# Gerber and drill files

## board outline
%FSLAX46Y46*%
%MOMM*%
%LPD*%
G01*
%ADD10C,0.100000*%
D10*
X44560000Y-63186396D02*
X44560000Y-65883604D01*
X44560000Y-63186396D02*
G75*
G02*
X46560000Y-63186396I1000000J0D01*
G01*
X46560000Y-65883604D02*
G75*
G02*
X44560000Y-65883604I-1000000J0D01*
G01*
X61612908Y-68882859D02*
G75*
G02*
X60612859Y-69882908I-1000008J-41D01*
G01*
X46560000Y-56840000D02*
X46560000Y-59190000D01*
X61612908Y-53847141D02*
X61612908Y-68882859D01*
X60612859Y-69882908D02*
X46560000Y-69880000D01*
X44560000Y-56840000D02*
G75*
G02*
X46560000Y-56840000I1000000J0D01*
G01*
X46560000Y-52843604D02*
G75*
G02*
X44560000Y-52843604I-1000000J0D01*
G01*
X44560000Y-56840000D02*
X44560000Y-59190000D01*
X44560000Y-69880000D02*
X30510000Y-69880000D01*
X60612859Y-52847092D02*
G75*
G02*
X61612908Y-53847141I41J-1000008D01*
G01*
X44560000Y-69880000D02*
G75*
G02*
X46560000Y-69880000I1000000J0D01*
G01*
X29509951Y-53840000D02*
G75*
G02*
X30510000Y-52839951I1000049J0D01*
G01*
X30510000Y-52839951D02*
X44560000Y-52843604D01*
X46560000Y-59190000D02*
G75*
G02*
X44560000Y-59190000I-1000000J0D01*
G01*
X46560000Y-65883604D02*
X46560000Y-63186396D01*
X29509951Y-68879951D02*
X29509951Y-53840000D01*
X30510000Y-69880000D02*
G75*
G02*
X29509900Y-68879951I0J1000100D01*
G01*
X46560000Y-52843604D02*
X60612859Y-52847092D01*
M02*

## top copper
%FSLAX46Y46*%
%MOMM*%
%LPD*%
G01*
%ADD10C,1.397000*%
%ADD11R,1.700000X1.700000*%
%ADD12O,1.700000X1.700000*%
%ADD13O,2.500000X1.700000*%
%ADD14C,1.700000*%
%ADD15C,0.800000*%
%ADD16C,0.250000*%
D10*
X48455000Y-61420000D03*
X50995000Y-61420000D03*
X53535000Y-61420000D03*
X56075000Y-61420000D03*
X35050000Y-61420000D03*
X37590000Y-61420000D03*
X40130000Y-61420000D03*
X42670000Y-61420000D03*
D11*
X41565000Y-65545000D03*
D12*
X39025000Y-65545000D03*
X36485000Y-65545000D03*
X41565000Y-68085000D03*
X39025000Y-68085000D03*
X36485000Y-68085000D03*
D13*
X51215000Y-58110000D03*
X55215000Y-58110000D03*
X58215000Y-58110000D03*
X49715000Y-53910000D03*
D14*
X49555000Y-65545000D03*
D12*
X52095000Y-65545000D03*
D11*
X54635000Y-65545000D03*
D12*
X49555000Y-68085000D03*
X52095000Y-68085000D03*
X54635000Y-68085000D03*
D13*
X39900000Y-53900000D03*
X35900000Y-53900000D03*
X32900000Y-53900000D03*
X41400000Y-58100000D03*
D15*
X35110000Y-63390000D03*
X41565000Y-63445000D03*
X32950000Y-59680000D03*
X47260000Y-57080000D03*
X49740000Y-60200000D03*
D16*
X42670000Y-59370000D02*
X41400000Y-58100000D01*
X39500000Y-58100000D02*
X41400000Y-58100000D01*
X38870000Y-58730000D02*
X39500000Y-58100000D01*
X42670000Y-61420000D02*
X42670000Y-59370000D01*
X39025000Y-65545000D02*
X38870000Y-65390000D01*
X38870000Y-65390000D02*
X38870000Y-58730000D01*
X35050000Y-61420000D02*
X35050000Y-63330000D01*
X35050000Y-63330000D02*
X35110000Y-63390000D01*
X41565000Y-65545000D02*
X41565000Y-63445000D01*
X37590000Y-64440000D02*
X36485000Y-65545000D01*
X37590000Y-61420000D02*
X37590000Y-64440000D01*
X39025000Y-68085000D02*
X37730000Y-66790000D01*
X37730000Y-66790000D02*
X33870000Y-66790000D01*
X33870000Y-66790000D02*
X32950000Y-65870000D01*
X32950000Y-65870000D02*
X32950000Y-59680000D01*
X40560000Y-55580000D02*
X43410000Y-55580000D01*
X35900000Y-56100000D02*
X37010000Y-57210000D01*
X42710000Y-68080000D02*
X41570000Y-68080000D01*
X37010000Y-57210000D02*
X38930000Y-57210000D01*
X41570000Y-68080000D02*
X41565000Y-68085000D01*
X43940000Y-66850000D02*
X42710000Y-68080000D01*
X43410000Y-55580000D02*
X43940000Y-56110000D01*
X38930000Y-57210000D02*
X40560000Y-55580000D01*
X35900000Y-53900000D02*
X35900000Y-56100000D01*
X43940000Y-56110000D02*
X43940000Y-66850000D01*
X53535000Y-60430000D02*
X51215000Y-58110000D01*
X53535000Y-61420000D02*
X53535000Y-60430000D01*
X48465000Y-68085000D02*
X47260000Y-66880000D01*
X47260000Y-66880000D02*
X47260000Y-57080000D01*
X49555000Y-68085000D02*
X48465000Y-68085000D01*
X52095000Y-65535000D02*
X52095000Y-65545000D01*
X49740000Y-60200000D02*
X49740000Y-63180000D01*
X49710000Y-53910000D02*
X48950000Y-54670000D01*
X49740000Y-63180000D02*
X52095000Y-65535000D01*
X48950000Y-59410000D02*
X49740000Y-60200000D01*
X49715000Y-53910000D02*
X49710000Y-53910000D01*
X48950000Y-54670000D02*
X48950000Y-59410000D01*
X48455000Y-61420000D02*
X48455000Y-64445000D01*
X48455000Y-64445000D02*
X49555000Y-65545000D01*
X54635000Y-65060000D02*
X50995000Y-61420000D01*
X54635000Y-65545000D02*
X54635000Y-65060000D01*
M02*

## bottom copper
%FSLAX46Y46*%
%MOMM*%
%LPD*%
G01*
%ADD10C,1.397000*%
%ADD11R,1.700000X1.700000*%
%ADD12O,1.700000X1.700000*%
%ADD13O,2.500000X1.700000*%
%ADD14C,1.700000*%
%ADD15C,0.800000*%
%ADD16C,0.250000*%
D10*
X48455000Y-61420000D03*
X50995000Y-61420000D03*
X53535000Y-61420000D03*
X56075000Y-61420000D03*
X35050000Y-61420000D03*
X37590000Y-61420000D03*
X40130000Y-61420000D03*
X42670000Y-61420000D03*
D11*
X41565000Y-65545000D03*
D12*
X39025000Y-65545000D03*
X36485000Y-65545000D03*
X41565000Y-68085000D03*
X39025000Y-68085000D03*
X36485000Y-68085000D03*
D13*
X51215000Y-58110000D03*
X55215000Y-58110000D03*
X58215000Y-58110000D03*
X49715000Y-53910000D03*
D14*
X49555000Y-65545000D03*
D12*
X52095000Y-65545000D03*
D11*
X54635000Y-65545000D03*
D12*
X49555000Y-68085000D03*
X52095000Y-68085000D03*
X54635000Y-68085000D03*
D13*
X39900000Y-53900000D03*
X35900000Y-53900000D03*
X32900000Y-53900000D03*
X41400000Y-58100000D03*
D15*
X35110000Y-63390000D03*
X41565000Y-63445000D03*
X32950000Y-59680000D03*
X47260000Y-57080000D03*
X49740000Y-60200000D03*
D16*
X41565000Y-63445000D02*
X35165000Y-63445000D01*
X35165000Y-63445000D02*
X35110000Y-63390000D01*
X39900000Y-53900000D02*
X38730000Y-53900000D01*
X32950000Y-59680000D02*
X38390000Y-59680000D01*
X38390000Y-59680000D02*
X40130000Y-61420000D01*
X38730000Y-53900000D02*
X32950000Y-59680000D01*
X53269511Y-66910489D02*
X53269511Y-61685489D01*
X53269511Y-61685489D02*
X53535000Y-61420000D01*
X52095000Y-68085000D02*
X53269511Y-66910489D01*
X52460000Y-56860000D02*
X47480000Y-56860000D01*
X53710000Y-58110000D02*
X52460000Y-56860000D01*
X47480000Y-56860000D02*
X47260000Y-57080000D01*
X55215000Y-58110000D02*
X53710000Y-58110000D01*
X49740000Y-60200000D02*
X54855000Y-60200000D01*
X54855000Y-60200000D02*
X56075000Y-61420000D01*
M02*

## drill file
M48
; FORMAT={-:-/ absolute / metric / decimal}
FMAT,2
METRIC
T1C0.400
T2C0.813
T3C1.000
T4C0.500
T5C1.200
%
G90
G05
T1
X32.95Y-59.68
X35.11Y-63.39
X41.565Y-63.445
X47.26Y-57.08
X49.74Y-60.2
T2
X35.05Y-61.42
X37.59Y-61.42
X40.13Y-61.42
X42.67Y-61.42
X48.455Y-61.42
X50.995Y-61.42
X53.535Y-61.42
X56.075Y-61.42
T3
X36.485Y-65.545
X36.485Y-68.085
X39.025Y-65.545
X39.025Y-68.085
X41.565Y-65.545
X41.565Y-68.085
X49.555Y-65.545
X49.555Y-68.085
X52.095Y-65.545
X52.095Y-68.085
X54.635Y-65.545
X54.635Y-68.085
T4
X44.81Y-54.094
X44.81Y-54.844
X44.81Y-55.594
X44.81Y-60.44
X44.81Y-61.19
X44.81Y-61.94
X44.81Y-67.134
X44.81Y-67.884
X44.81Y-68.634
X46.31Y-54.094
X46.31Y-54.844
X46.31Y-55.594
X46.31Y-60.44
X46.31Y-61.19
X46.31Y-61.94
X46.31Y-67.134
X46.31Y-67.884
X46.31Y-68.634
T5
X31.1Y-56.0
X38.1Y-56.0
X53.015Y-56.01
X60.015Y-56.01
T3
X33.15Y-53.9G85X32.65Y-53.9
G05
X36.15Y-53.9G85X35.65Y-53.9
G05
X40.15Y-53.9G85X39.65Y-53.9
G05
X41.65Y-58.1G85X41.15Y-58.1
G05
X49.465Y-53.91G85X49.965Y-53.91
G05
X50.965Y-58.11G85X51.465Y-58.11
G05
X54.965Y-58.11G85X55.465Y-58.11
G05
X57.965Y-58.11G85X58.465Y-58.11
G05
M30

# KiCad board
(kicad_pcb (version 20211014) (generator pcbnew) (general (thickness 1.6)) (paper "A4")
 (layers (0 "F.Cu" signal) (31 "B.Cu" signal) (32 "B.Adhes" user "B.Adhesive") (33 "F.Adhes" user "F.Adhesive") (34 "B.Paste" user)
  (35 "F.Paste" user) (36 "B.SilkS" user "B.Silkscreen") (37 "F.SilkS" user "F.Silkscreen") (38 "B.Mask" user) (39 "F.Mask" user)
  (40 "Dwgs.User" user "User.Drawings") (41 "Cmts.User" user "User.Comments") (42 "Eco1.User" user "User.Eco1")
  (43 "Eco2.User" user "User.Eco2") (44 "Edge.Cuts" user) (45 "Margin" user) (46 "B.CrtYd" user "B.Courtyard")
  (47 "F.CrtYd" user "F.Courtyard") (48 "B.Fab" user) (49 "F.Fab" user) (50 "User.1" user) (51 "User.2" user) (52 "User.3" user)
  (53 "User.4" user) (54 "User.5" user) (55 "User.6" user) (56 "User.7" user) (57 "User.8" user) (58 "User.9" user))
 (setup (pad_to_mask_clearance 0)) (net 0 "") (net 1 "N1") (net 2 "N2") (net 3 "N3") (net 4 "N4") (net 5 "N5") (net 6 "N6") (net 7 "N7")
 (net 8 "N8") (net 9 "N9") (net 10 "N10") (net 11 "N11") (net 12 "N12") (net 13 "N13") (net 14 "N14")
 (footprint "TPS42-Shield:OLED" (layer "F.Cu") (at 52.265 61.42)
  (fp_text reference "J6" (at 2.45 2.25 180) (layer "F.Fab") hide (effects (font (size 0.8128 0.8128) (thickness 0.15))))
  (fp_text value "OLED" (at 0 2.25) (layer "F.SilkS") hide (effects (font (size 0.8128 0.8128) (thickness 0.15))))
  (pad "1" thru_hole circle (at -3.81 0) (size 1.397 1.397) (drill 0.8128) (layers *.Cu *.Mask "F.SilkS") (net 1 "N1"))
  (pad "2" thru_hole circle (at -1.27 0) (size 1.397 1.397) (drill 0.8128) (layers *.Cu *.Mask "F.SilkS") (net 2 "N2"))
  (pad "3" thru_hole circle (at 1.27 0) (size 1.397 1.397) (drill 0.8128) (layers *.Cu *.Mask "F.SilkS") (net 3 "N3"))
  (pad "4" thru_hole circle (at 3.81 0) (size 1.397 1.397) (drill 0.8128) (layers *.Cu *.Mask "F.SilkS") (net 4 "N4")))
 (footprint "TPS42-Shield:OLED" (layer "F.Cu") (at 38.86 61.42)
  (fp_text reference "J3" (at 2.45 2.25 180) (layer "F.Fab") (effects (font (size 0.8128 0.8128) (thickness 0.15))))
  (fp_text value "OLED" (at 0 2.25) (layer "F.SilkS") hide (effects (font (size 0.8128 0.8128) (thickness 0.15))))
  (pad "1" thru_hole circle (at -3.81 0) (size 1.397 1.397) (drill 0.8128) (layers *.Cu *.Mask "F.SilkS") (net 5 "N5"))
  (pad "2" thru_hole circle (at -1.27 0) (size 1.397 1.397) (drill 0.8128) (layers *.Cu *.Mask "F.SilkS") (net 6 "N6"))
  (pad "3" thru_hole circle (at 1.27 0) (size 1.397 1.397) (drill 0.8128) (layers *.Cu *.Mask "F.SilkS") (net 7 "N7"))
  (pad "4" thru_hole circle (at 3.81 0) (size 1.397 1.397) (drill 0.8128) (layers *.Cu *.Mask "F.SilkS") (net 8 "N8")))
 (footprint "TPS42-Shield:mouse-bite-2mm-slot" (layer "F.Cu") (at 45.56 67.883604 90)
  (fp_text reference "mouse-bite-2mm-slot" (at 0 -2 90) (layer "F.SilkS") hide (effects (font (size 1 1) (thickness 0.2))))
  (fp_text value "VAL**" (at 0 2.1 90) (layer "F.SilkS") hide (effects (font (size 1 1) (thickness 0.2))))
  (pad "" np_thru_hole circle (at -0.75 0.75 90) (size 0.5 0.5) (drill 0.5) (layers *.Cu *.Mask))
  (pad "" np_thru_hole circle (at 0.75 -0.75 90) (size 0.5 0.5) (drill 0.5) (layers *.Cu *.Mask))
  (pad "" np_thru_hole circle (at -0.75 -0.75 90) (size 0.5 0.5) (drill 0.5) (layers *.Cu *.Mask))
  (pad "" np_thru_hole circle (at 0 -0.75 90) (size 0.5 0.5) (drill 0.5) (layers *.Cu *.Mask))
  (pad "" np_thru_hole circle (at 0.75 0.75 90) (size 0.5 0.5) (drill 0.5) (layers *.Cu *.Mask))
  (pad "" np_thru_hole circle (at 0 0.75 90) (size 0.5 0.5) (drill 0.5) (layers *.Cu *.Mask)))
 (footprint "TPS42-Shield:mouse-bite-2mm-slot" (layer "F.Cu") (at 45.56 61.19 90)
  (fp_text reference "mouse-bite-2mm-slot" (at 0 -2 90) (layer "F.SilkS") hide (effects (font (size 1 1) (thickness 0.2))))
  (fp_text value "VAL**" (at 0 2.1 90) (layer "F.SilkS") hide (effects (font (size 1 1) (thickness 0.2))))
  (pad "" np_thru_hole circle (at -0.75 0.75 90) (size 0.5 0.5) (drill 0.5) (layers *.Cu *.Mask))
  (pad "" np_thru_hole circle (at 0.75 -0.75 90) (size 0.5 0.5) (drill 0.5) (layers *.Cu *.Mask))
  (pad "" np_thru_hole circle (at -0.75 -0.75 90) (size 0.5 0.5) (drill 0.5) (layers *.Cu *.Mask))
  (pad "" np_thru_hole circle (at 0 -0.75 90) (size 0.5 0.5) (drill 0.5) (layers *.Cu *.Mask))
  (pad "" np_thru_hole circle (at 0.75 0.75 90) (size 0.5 0.5) (drill 0.5) (layers *.Cu *.Mask))
  (pad "" np_thru_hole circle (at 0 0.75 90) (size 0.5 0.5) (drill 0.5) (layers *.Cu *.Mask)))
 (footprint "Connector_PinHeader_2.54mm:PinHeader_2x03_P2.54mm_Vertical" (layer "F.Cu") (at 41.565 65.545 -90)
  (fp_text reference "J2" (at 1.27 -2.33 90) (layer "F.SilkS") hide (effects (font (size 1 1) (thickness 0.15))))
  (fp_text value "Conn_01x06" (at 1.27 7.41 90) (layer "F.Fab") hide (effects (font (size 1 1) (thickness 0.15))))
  (pad "1" thru_hole rect (at 0 0 270) (size 1.7 1.7) (drill 1) (layers *.Cu *.Mask) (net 5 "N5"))
  (pad "2" thru_hole oval (at 0 2.54 270) (size 1.7 1.7) (drill 1) (layers *.Cu *.Mask) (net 8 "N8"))
  (pad "3" thru_hole oval (at 0 5.08 270) (size 1.7 1.7) (drill 1) (layers *.Cu *.Mask) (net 6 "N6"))
  (pad "4" thru_hole oval (at 2.54 0 270) (size 1.7 1.7) (drill 1) (layers *.Cu *.Mask) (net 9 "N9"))
  (pad "5" thru_hole oval (at 2.54 2.54 270) (size 1.7 1.7) (drill 1) (layers *.Cu *.Mask) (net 7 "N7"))
  (pad "6" thru_hole oval (at 2.54 5.08 270) (size 1.7 1.7) (drill 1) (layers *.Cu *.Mask) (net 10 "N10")))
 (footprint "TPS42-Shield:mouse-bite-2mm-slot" (layer "F.Cu") (at 45.56 54.843604 90)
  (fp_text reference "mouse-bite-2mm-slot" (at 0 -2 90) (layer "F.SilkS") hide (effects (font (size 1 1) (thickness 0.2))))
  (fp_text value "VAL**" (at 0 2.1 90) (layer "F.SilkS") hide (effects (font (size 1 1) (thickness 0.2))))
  (pad "" np_thru_hole circle (at -0.75 0.75 90) (size 0.5 0.5) (drill 0.5) (layers *.Cu *.Mask))
  (pad "" np_thru_hole circle (at 0.75 -0.75 90) (size 0.5 0.5) (drill 0.5) (layers *.Cu *.Mask))
  (pad "" np_thru_hole circle (at -0.75 -0.75 90) (size 0.5 0.5) (drill 0.5) (layers *.Cu *.Mask))
  (pad "" np_thru_hole circle (at 0 -0.75 90) (size 0.5 0.5) (drill 0.5) (layers *.Cu *.Mask))
  (pad "" np_thru_hole circle (at 0.75 0.75 90) (size 0.5 0.5) (drill 0.5) (layers *.Cu *.Mask))
  (pad "" np_thru_hole circle (at 0 0.75 90) (size 0.5 0.5) (drill 0.5) (layers *.Cu *.Mask)))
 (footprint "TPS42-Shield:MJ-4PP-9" (layer "B.Cu") (at 61.515 54.26 90)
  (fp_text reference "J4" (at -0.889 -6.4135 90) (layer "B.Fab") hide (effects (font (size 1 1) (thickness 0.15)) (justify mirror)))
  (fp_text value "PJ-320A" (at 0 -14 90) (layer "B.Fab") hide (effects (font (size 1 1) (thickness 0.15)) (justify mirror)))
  (pad "" np_thru_hole circle (at -1.75 -1.5 90) (size 1.2 1.2) (drill 1.2) (layers *.Cu *.Mask "B.SilkS"))
  (pad "" np_thru_hole circle (at -1.75 -8.5 90) (size 1.2 1.2) (drill 1.2) (layers *.Cu *.Mask "B.SilkS"))
  (pad "1" thru_hole oval (at -3.85 -10.3 90) (size 1.7 2.5) (drill oval 1 1.5) (layers *.Cu *.Mask "B.SilkS") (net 3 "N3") (clearance 0.15))
  (pad "2" thru_hole oval (at -3.85 -6.3 90) (size 1.7 2.5) (drill oval 1 1.5) (layers *.Cu *.Mask "B.SilkS") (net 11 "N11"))
  (pad "3" thru_hole oval (at -3.85 -3.3 90) (size 1.7 2.5) (drill oval 1 1.5) (layers *.Cu *.Mask "B.SilkS") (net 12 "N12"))
  (pad "4" thru_hole oval (at 0.35 -11.8 90) (size 1.7 2.5) (drill oval 1 1.5) (layers *.Cu *.Mask "B.SilkS") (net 4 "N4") (clearance 0.15)))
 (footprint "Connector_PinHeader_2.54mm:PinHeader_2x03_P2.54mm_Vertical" (layer "B.Cu") (at 49.555 65.545 -90)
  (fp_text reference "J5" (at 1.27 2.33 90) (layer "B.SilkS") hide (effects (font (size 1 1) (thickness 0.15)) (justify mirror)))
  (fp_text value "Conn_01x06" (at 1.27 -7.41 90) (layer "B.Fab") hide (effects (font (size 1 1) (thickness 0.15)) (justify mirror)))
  (pad "1" thru_hole circle (at 0 0 270) (size 1.7 1.7) (drill 1) (layers *.Cu *.Mask) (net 1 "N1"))
  (pad "2" thru_hole oval (at 0 -2.54 270) (size 1.7 1.7) (drill 1) (layers *.Cu *.Mask) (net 4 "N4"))
  (pad "3" thru_hole rect (at 0 -5.08 270) (size 1.7 1.7) (drill 1) (layers *.Cu *.Mask) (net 2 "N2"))
  (pad "4" thru_hole oval (at 2.54 0 270) (size 1.7 1.7) (drill 1) (layers *.Cu *.Mask) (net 11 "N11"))
  (pad "5" thru_hole oval (at 2.54 -2.54 270) (size 1.7 1.7) (drill 1) (layers *.Cu *.Mask) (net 3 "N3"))
  (pad "6" thru_hole oval (at 2.54 -5.08 270) (size 1.7 1.7) (drill 1) (layers *.Cu *.Mask) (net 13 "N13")))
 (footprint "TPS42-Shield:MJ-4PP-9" (layer "B.Cu") (at 29.6 57.75 -90)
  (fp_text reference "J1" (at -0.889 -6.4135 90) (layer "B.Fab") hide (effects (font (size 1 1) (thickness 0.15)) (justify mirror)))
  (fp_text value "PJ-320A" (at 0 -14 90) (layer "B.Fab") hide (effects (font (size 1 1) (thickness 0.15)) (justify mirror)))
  (pad "" np_thru_hole circle (at -1.75 -1.5 270) (size 1.2 1.2) (drill 1.2) (layers *.Cu *.Mask "B.SilkS"))
  (pad "" np_thru_hole circle (at -1.75 -8.5 270) (size 1.2 1.2) (drill 1.2) (layers *.Cu *.Mask "B.SilkS"))
  (pad "1" thru_hole oval (at -3.85 -10.3 270) (size 1.7 2.5) (drill oval 1 1.5) (layers *.Cu *.Mask "B.SilkS") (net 7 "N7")
   (clearance 0.15))
  (pad "2" thru_hole oval (at -3.85 -6.3 270) (size 1.7 2.5) (drill oval 1 1.5) (layers *.Cu *.Mask "B.SilkS") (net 9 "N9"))
  (pad "3" thru_hole oval (at -3.85 -3.3 270) (size 1.7 2.5) (drill oval 1 1.5) (layers *.Cu *.Mask "B.SilkS") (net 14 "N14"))
  (pad "4" thru_hole oval (at 0.35 -11.8 270) (size 1.7 2.5) (drill oval 1 1.5) (layers *.Cu *.Mask "B.SilkS") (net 8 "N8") (clearance 0.15)))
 (gr_line (start 44.56 63.186396) (end 44.56 65.883604) (layer "Edge.Cuts") (width 0.1))
 (gr_arc (start 44.56 63.186396) (mid 45.56 62.186396) (end 46.56 63.186396) (layer "Edge.Cuts") (width 0.1))
 (gr_arc (start 46.56 65.883604) (mid 45.56 66.883604) (end 44.56 65.883604) (layer "Edge.Cuts") (width 0.1))
 (gr_arc (start 61.612908 68.882859) (mid 61.32 69.59) (end 60.612859 69.882908) (layer "Edge.Cuts") (width 0.1))
 (gr_line (start 46.56 56.84) (end 46.56 59.19) (layer "Edge.Cuts") (width 0.1))
 (gr_line (start 61.612908 53.847141) (end 61.612908 68.882859) (layer "Edge.Cuts") (width 0.1))
 (gr_line (start 60.612859 69.882908) (end 46.56 69.88) (layer "Edge.Cuts") (width 0.1))
 (gr_arc (start 44.56 56.84) (mid 45.56 55.84) (end 46.56 56.84) (layer "Edge.Cuts") (width 0.1))
 (gr_arc (start 46.56 52.843604) (mid 45.56 53.843604) (end 44.56 52.843604) (layer "Edge.Cuts") (width 0.1))
 (gr_line (start 44.56 56.84) (end 44.56 59.19) (layer "Edge.Cuts") (width 0.1))
 (gr_line (start 44.56 69.88) (end 30.51 69.88) (layer "Edge.Cuts") (width 0.1))
 (gr_arc (start 60.612859 52.847092) (mid 61.32 53.14) (end 61.612908 53.847141) (layer "Edge.Cuts") (width 0.1))
 (gr_arc (start 44.56 69.88) (mid 45.56 68.88) (end 46.56 69.88) (layer "Edge.Cuts") (width 0.1))
 (gr_arc (start 29.509951 53.84) (mid 29.802859 53.132859) (end 30.51 52.839951) (layer "Edge.Cuts") (width 0.1))
 (gr_line (start 30.51 52.839951) (end 44.56 52.843604) (layer "Edge.Cuts") (width 0.1))
 (gr_arc (start 46.56 59.19) (mid 45.56 60.19) (end 44.56 59.19) (layer "Edge.Cuts") (width 0.1))
 (gr_line (start 46.56 65.883604) (end 46.56 63.186396) (layer "Edge.Cuts") (width 0.1))
 (gr_line (start 29.509951 68.879951) (end 29.509951 53.84) (layer "Edge.Cuts") (width 0.1))
 (gr_arc (start 30.51 69.88) (mid 29.802859 69.587092) (end 29.509951 68.879951) (layer "Edge.Cuts") (width 0.1))
 (gr_line (start 46.56 52.843604) (end 60.612859 52.847092) (layer "Edge.Cuts") (width 0.1))
 (segment (start 42.67 59.37) (end 41.4 58.1) (width 0.25) (layer "F.Cu") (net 8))
 (segment (start 39.5 58.1) (end 41.4 58.1) (width 0.25) (layer "F.Cu") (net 8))
 (segment (start 38.87 58.73) (end 39.5 58.1) (width 0.25) (layer "F.Cu") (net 8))
 (segment (start 42.67 61.42) (end 42.67 59.37) (width 0.25) (layer "F.Cu") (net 8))
 (segment (start 39.025 65.545) (end 38.87 65.39) (width 0.25) (layer "F.Cu") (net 8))
 (segment (start 38.87 65.39) (end 38.87 58.73) (width 0.25) (layer "F.Cu") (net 8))
 (segment (start 35.05 61.42) (end 35.05 63.33) (width 0.25) (layer "F.Cu") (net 5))
 (segment (start 35.05 63.33) (end 35.11 63.39) (width 0.25) (layer "F.Cu") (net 5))
 (segment (start 41.565 65.545) (end 41.565 63.445) (width 0.25) (layer "F.Cu") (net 5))
 (via (at 35.11 63.39) (size 0.8) (drill 0.4) (layers "F.Cu" "B.Cu") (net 5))
 (via (at 41.565 63.445) (size 0.8) (drill 0.4) (layers "F.Cu" "B.Cu") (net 5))
 (segment (start 41.565 63.445) (end 35.165 63.445) (width 0.25) (layer "B.Cu") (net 5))
 (segment (start 35.165 63.445) (end 35.11 63.39) (width 0.25) (layer "B.Cu") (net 5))
 (segment (start 37.59 64.44) (end 36.485 65.545) (width 0.25) (layer "F.Cu") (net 6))
 (segment (start 37.59 61.42) (end 37.59 64.44) (width 0.25) (layer "F.Cu") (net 6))
 (segment (start 39.025 68.085) (end 37.73 66.79) (width 0.25) (layer "F.Cu") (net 7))
 (segment (start 37.73 66.79) (end 33.87 66.79) (width 0.25) (layer "F.Cu") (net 7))
 (segment (start 33.87 66.79) (end 32.95 65.87) (width 0.25) (layer "F.Cu") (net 7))
 (segment (start 32.95 65.87) (end 32.95 59.68) (width 0.25) (layer "F.Cu") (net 7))
 (via (at 32.95 59.68) (size 0.8) (drill 0.4) (layers "F.Cu" "B.Cu") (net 7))
 (segment (start 39.9 53.9) (end 38.73 53.9) (width 0.25) (layer "B.Cu") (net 7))
 (segment (start 32.95 59.68) (end 38.39 59.68) (width 0.25) (layer "B.Cu") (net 7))
 (segment (start 38.39 59.68) (end 40.13 61.42) (width 0.25) (layer "B.Cu") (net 7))
 (segment (start 38.73 53.9) (end 32.95 59.68) (width 0.25) (layer "B.Cu") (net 7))
 (segment (start 40.56 55.58) (end 43.41 55.58) (width 0.25) (layer "F.Cu") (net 9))
 (segment (start 35.9 56.1) (end 37.01 57.21) (width 0.25) (layer "F.Cu") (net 9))
 (segment (start 42.71 68.08) (end 41.57 68.08) (width 0.25) (layer "F.Cu") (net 9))
 (segment (start 37.01 57.21) (end 38.93 57.21) (width 0.25) (layer "F.Cu") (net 9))
 (segment (start 41.57 68.08) (end 41.565 68.085) (width 0.25) (layer "F.Cu") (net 9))
 (segment (start 43.94 66.85) (end 42.71 68.08) (width 0.25) (layer "F.Cu") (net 9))
 (segment (start 43.41 55.58) (end 43.94 56.11) (width 0.25) (layer "F.Cu") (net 9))
 (segment (start 38.93 57.21) (end 40.56 55.58) (width 0.25) (layer "F.Cu") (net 9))
 (segment (start 35.9 53.9) (end 35.9 56.1) (width 0.25) (layer "F.Cu") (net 9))
 (segment (start 43.94 56.11) (end 43.94 66.85) (width 0.25) (layer "F.Cu") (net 9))
 (segment (start 53.535 60.43) (end 51.215 58.11) (width 0.25) (layer "F.Cu") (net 3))
 (segment (start 53.535 61.42) (end 53.535 60.43) (width 0.25) (layer "F.Cu") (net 3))
 (segment (start 53.269511 66.910489) (end 53.269511 61.685489) (width 0.25) (layer "B.Cu") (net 3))
 (segment (start 53.269511 61.685489) (end 53.535 61.42) (width 0.25) (layer "B.Cu") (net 3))
 (segment (start 52.095 68.085) (end 53.269511 66.910489) (width 0.25) (layer "B.Cu") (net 3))
 (segment (start 48.465 68.085) (end 47.26 66.88) (width 0.25) (layer "F.Cu") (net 11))
 (segment (start 47.26 66.88) (end 47.26 57.08) (width 0.25) (layer "F.Cu") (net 11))
 (segment (start 49.555 68.085) (end 48.465 68.085) (width 0.25) (layer "F.Cu") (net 11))
 (via (at 47.26 57.08) (size 0.8) (drill 0.4) (layers "F.Cu" "B.Cu") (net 11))
 (segment (start 52.46 56.86) (end 47.48 56.86) (width 0.25) (layer "B.Cu") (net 11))
 (segment (start 53.71 58.11) (end 52.46 56.86) (width 0.25) (layer "B.Cu") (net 11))
 (segment (start 47.48 56.86) (end 47.26 57.08) (width 0.25) (layer "B.Cu") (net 11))
 (segment (start 55.215 58.11) (end 53.71 58.11) (width 0.25) (layer "B.Cu") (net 11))
 (segment (start 52.095 65.535) (end 52.095 65.545) (width 0.25) (layer "F.Cu") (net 4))
 (segment (start 49.74 60.2) (end 49.74 63.18) (width 0.25) (layer "F.Cu") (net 4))
 (segment (start 49.71 53.91) (end 48.95 54.67) (width 0.25) (layer "F.Cu") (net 4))
 (segment (start 49.74 63.18) (end 52.095 65.535) (width 0.25) (layer "F.Cu") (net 4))
 (segment (start 48.95 59.41) (end 49.74 60.2) (width 0.25) (layer "F.Cu") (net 4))
 (segment (start 49.715 53.91) (end 49.71 53.91) (width 0.25) (layer "F.Cu") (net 4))
 (segment (start 48.95 54.67) (end 48.95 59.41) (width 0.25) (layer "F.Cu") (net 4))
 (via (at 49.74 60.2) (size 0.8) (drill 0.4) (layers "F.Cu" "B.Cu") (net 4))
 (segment (start 49.74 60.2) (end 54.855 60.2) (width 0.25) (layer "B.Cu") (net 4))
 (segment (start 54.855 60.2) (end 56.075 61.42) (width 0.25) (layer "B.Cu") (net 4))
 (segment (start 48.455 61.42) (end 48.455 64.445) (width 0.25) (layer "F.Cu") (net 1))
 (segment (start 48.455 64.445) (end 49.555 65.545) (width 0.25) (layer "F.Cu") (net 1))
 (segment (start 54.635 65.06) (end 50.995 61.42) (width 0.25) (layer "F.Cu") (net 2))
 (segment (start 54.635 65.545) (end 54.635 65.06) (width 0.25) (layer "F.Cu") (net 2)))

